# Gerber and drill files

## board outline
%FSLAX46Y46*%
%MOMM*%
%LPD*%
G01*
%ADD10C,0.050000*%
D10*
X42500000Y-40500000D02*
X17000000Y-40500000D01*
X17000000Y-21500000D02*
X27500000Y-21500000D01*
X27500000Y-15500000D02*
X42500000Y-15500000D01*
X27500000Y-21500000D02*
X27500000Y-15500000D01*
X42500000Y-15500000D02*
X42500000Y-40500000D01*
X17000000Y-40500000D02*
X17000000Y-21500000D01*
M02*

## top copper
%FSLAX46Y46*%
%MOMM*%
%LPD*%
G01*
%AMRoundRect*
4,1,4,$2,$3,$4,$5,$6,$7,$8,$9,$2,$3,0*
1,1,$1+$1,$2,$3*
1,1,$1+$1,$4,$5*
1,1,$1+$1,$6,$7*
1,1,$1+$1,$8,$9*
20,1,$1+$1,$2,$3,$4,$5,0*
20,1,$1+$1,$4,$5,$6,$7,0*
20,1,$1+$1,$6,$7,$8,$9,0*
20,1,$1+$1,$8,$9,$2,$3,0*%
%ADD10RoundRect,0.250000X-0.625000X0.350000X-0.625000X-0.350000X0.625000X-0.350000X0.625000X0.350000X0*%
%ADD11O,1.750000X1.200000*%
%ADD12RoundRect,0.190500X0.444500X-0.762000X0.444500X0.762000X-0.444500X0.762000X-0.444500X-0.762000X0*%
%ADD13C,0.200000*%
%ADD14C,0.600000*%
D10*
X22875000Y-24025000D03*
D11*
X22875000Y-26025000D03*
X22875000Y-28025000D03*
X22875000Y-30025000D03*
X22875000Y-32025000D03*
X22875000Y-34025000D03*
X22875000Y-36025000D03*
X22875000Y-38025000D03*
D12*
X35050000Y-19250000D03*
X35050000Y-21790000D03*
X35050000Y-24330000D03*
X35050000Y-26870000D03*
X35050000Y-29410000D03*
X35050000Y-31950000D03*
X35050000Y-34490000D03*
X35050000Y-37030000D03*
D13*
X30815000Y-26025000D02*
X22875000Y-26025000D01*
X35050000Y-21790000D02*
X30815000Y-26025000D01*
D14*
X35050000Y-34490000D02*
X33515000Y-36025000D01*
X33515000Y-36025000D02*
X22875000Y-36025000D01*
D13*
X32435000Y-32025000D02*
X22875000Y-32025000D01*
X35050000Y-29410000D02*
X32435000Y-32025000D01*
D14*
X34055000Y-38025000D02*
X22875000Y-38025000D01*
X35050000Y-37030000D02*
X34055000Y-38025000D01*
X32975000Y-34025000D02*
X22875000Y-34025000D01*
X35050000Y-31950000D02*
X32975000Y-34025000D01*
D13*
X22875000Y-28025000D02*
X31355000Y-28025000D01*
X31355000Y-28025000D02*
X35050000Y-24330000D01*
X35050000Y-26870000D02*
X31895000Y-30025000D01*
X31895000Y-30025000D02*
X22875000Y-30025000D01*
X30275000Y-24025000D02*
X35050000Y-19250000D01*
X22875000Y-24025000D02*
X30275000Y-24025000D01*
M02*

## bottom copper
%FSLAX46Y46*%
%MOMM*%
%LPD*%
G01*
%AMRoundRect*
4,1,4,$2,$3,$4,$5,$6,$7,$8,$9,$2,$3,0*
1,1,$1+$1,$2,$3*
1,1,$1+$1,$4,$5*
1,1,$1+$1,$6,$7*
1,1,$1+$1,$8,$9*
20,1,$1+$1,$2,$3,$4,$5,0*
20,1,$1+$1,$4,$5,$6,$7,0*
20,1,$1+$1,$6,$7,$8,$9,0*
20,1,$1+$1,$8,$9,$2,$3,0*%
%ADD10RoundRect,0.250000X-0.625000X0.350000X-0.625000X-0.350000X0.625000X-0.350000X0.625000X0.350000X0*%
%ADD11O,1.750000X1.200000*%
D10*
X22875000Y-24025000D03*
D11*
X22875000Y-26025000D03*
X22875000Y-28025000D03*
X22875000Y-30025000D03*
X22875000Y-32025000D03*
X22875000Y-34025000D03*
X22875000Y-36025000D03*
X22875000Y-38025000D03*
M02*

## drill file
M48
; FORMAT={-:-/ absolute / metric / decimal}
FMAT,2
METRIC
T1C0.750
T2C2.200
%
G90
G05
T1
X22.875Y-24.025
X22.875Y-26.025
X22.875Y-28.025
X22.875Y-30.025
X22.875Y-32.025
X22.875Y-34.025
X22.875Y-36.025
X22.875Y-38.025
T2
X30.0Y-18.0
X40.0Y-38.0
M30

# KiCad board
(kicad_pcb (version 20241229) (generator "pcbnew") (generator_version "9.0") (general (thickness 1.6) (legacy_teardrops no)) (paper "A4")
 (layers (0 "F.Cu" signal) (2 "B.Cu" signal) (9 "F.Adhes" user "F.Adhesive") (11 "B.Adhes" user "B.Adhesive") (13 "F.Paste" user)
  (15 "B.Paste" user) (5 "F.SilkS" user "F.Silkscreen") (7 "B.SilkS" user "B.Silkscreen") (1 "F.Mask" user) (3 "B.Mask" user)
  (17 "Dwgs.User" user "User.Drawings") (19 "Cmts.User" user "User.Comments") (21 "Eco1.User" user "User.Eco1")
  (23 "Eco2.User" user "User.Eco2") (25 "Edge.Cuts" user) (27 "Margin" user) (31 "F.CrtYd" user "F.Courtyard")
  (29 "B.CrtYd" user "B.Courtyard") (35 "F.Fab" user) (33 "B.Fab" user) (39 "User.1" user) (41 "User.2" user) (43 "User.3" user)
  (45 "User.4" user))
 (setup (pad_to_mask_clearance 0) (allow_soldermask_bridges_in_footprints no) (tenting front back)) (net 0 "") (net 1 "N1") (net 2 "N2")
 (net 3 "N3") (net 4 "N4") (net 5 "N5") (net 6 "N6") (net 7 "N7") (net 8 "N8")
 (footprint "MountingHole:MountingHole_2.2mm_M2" (layer "F.Cu") (at 40 38)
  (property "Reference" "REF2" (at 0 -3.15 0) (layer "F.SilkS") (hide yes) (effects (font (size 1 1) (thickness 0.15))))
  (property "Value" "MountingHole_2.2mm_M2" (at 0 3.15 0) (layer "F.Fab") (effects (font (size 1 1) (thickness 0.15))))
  (pad "" np_thru_hole circle (at 0 0) (size 2.2 2.2) (drill 2.2) (layers "*.Cu" "*.Mask")))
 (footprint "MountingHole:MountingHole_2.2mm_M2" (layer "F.Cu") (at 30 18)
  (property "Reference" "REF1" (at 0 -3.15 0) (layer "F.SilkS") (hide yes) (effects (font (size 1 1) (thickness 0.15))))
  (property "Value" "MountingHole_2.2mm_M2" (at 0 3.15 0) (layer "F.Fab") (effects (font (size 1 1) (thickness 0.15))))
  (pad "" np_thru_hole circle (at 0 0) (size 2.2 2.2) (drill 2.2) (layers "*.Cu" "*.Mask")))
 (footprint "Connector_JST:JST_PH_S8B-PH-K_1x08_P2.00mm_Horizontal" (layer "F.Cu") (at 22.875 24.025 -90)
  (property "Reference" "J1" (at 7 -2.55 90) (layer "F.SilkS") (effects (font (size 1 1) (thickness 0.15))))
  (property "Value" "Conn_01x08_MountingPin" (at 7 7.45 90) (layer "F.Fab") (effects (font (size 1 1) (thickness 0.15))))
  (pad "1" thru_hole roundrect (at 0 0 270) (size 1.2 1.75) (drill 0.75) (layers "*.Cu" "*.Mask") (remove_unused_layers no)
   (roundrect_rratio 0.208333) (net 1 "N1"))
  (pad "2" thru_hole oval (at 2 0 270) (size 1.2 1.75) (drill 0.75) (layers "*.Cu" "*.Mask") (remove_unused_layers no) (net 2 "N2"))
  (pad "3" thru_hole oval (at 4 0 270) (size 1.2 1.75) (drill 0.75) (layers "*.Cu" "*.Mask") (remove_unused_layers no) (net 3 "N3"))
  (pad "4" thru_hole oval (at 6 0 270) (size 1.2 1.75) (drill 0.75) (layers "*.Cu" "*.Mask") (remove_unused_layers no) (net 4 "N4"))
  (pad "5" thru_hole oval (at 8 0 270) (size 1.2 1.75) (drill 0.75) (layers "*.Cu" "*.Mask") (remove_unused_layers no) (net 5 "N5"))
  (pad "6" thru_hole oval (at 10 0 270) (size 1.2 1.75) (drill 0.75) (layers "*.Cu" "*.Mask") (remove_unused_layers no) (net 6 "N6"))
  (pad "7" thru_hole oval (at 12 0 270) (size 1.2 1.75) (drill 0.75) (layers "*.Cu" "*.Mask") (remove_unused_layers no) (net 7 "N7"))
  (pad "8" thru_hole oval (at 14 0 270) (size 1.2 1.75) (drill 0.75) (layers "*.Cu" "*.Mask") (remove_unused_layers no) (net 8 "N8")))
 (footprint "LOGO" (layer "F.Cu") (at 29 30)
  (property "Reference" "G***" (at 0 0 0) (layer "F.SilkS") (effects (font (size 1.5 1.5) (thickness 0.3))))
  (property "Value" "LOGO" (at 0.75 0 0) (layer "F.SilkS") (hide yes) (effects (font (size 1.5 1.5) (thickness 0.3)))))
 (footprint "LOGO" (layer "F.Cu") (at 38.5 19.5 -90)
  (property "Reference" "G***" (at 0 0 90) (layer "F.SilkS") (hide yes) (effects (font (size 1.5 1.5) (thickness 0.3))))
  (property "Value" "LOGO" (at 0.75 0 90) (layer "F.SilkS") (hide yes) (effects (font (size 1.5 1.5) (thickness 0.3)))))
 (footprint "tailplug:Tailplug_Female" (layer "F.Cu") (at 35.05 15.25)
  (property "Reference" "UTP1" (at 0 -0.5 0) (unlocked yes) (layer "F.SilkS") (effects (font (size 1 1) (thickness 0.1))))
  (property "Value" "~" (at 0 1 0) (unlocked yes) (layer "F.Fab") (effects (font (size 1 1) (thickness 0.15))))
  (pad "1" smd roundrect (at 0 4 90) (size 1.905 1.27) (layers "F.Cu" "F.Mask" "F.Paste") (roundrect_rratio 0.15) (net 1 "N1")
   (thermal_bridge_angle 45))
  (pad "2" smd roundrect (at 0 6.54 90) (size 1.905 1.27) (layers "F.Cu" "F.Mask" "F.Paste") (roundrect_rratio 0.15) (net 2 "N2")
   (thermal_bridge_angle 45))
  (pad "3" smd roundrect (at 0 9.08 90) (size 1.905 1.27) (layers "F.Cu" "F.Mask" "F.Paste") (roundrect_rratio 0.15) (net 3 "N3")
   (thermal_bridge_angle 45))
  (pad "4" smd roundrect (at 0 11.62 90) (size 1.905 1.27) (layers "F.Cu" "F.Mask" "F.Paste") (roundrect_rratio 0.15) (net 4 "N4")
   (thermal_bridge_angle 45))
  (pad "5" smd roundrect (at 0 14.16 90) (size 1.905 1.27) (layers "F.Cu" "F.Mask" "F.Paste") (roundrect_rratio 0.15) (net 5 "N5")
   (thermal_bridge_angle 45))
  (pad "6" smd roundrect (at 0 16.7 90) (size 1.905 1.27) (layers "F.Cu" "F.Mask" "F.Paste") (roundrect_rratio 0.15) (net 6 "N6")
   (thermal_bridge_angle 45))
  (pad "7" smd roundrect (at 0 19.24 90) (size 1.905 1.27) (layers "F.Cu" "F.Mask" "F.Paste") (roundrect_rratio 0.15) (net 7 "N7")
   (thermal_bridge_angle 45))
  (pad "8" smd roundrect (at 0 21.78 90) (size 1.905 1.27) (layers "F.Cu" "F.Mask" "F.Paste") (roundrect_rratio 0.15) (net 8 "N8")
   (thermal_bridge_angle 45)))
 (gr_line (start 42.5 40.5) (end 17 40.5) (stroke (width 0.05) (type default)) (layer "Edge.Cuts"))
 (gr_line (start 17 21.5) (end 27.5 21.5) (stroke (width 0.05) (type default)) (layer "Edge.Cuts"))
 (gr_line (start 27.5 15.5) (end 42.5 15.5) (stroke (width 0.05) (type default)) (layer "Edge.Cuts"))
 (gr_line (start 27.5 21.5) (end 27.5 15.5) (stroke (width 0.05) (type default)) (layer "Edge.Cuts"))
 (gr_line (start 42.5 15.5) (end 42.5 40.5) (stroke (width 0.05) (type default)) (layer "Edge.Cuts"))
 (gr_line (start 17 40.5) (end 17 21.5) (stroke (width 0.05) (type default)) (layer "Edge.Cuts"))
 (segment (start 30.815 26.025) (end 22.875 26.025) (width 0.2) (layer "F.Cu") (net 2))
 (segment (start 35.05 21.79) (end 30.815 26.025) (width 0.2) (layer "F.Cu") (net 2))
 (segment (start 35.05 34.49) (end 33.515 36.025) (width 0.6) (layer "F.Cu") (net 7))
 (segment (start 33.515 36.025) (end 22.875 36.025) (width 0.6) (layer "F.Cu") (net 7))
 (segment (start 32.435 32.025) (end 22.875 32.025) (width 0.2) (layer "F.Cu") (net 5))
 (segment (start 35.05 29.41) (end 32.435 32.025) (width 0.2) (layer "F.Cu") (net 5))
 (segment (start 34.055 38.025) (end 22.875 38.025) (width 0.6) (layer "F.Cu") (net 8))
 (segment (start 35.05 37.03) (end 34.055 38.025) (width 0.6) (layer "F.Cu") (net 8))
 (segment (start 32.975 34.025) (end 22.875 34.025) (width 0.6) (layer "F.Cu") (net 6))
 (segment (start 35.05 31.95) (end 32.975 34.025) (width 0.6) (layer "F.Cu") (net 6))
 (segment (start 22.875 28.025) (end 31.355 28.025) (width 0.2) (layer "F.Cu") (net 3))
 (segment (start 31.355 28.025) (end 35.05 24.33) (width 0.2) (layer "F.Cu") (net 3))
 (segment (start 35.05 26.87) (end 31.895 30.025) (width 0.2) (layer "F.Cu") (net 4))
 (segment (start 31.895 30.025) (end 22.875 30.025) (width 0.2) (layer "F.Cu") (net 4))
 (segment (start 30.275 24.025) (end 35.05 19.25) (width 0.2) (layer "F.Cu") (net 1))
 (segment (start 22.875 24.025) (end 30.275 24.025) (width 0.2) (layer "F.Cu") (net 1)))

